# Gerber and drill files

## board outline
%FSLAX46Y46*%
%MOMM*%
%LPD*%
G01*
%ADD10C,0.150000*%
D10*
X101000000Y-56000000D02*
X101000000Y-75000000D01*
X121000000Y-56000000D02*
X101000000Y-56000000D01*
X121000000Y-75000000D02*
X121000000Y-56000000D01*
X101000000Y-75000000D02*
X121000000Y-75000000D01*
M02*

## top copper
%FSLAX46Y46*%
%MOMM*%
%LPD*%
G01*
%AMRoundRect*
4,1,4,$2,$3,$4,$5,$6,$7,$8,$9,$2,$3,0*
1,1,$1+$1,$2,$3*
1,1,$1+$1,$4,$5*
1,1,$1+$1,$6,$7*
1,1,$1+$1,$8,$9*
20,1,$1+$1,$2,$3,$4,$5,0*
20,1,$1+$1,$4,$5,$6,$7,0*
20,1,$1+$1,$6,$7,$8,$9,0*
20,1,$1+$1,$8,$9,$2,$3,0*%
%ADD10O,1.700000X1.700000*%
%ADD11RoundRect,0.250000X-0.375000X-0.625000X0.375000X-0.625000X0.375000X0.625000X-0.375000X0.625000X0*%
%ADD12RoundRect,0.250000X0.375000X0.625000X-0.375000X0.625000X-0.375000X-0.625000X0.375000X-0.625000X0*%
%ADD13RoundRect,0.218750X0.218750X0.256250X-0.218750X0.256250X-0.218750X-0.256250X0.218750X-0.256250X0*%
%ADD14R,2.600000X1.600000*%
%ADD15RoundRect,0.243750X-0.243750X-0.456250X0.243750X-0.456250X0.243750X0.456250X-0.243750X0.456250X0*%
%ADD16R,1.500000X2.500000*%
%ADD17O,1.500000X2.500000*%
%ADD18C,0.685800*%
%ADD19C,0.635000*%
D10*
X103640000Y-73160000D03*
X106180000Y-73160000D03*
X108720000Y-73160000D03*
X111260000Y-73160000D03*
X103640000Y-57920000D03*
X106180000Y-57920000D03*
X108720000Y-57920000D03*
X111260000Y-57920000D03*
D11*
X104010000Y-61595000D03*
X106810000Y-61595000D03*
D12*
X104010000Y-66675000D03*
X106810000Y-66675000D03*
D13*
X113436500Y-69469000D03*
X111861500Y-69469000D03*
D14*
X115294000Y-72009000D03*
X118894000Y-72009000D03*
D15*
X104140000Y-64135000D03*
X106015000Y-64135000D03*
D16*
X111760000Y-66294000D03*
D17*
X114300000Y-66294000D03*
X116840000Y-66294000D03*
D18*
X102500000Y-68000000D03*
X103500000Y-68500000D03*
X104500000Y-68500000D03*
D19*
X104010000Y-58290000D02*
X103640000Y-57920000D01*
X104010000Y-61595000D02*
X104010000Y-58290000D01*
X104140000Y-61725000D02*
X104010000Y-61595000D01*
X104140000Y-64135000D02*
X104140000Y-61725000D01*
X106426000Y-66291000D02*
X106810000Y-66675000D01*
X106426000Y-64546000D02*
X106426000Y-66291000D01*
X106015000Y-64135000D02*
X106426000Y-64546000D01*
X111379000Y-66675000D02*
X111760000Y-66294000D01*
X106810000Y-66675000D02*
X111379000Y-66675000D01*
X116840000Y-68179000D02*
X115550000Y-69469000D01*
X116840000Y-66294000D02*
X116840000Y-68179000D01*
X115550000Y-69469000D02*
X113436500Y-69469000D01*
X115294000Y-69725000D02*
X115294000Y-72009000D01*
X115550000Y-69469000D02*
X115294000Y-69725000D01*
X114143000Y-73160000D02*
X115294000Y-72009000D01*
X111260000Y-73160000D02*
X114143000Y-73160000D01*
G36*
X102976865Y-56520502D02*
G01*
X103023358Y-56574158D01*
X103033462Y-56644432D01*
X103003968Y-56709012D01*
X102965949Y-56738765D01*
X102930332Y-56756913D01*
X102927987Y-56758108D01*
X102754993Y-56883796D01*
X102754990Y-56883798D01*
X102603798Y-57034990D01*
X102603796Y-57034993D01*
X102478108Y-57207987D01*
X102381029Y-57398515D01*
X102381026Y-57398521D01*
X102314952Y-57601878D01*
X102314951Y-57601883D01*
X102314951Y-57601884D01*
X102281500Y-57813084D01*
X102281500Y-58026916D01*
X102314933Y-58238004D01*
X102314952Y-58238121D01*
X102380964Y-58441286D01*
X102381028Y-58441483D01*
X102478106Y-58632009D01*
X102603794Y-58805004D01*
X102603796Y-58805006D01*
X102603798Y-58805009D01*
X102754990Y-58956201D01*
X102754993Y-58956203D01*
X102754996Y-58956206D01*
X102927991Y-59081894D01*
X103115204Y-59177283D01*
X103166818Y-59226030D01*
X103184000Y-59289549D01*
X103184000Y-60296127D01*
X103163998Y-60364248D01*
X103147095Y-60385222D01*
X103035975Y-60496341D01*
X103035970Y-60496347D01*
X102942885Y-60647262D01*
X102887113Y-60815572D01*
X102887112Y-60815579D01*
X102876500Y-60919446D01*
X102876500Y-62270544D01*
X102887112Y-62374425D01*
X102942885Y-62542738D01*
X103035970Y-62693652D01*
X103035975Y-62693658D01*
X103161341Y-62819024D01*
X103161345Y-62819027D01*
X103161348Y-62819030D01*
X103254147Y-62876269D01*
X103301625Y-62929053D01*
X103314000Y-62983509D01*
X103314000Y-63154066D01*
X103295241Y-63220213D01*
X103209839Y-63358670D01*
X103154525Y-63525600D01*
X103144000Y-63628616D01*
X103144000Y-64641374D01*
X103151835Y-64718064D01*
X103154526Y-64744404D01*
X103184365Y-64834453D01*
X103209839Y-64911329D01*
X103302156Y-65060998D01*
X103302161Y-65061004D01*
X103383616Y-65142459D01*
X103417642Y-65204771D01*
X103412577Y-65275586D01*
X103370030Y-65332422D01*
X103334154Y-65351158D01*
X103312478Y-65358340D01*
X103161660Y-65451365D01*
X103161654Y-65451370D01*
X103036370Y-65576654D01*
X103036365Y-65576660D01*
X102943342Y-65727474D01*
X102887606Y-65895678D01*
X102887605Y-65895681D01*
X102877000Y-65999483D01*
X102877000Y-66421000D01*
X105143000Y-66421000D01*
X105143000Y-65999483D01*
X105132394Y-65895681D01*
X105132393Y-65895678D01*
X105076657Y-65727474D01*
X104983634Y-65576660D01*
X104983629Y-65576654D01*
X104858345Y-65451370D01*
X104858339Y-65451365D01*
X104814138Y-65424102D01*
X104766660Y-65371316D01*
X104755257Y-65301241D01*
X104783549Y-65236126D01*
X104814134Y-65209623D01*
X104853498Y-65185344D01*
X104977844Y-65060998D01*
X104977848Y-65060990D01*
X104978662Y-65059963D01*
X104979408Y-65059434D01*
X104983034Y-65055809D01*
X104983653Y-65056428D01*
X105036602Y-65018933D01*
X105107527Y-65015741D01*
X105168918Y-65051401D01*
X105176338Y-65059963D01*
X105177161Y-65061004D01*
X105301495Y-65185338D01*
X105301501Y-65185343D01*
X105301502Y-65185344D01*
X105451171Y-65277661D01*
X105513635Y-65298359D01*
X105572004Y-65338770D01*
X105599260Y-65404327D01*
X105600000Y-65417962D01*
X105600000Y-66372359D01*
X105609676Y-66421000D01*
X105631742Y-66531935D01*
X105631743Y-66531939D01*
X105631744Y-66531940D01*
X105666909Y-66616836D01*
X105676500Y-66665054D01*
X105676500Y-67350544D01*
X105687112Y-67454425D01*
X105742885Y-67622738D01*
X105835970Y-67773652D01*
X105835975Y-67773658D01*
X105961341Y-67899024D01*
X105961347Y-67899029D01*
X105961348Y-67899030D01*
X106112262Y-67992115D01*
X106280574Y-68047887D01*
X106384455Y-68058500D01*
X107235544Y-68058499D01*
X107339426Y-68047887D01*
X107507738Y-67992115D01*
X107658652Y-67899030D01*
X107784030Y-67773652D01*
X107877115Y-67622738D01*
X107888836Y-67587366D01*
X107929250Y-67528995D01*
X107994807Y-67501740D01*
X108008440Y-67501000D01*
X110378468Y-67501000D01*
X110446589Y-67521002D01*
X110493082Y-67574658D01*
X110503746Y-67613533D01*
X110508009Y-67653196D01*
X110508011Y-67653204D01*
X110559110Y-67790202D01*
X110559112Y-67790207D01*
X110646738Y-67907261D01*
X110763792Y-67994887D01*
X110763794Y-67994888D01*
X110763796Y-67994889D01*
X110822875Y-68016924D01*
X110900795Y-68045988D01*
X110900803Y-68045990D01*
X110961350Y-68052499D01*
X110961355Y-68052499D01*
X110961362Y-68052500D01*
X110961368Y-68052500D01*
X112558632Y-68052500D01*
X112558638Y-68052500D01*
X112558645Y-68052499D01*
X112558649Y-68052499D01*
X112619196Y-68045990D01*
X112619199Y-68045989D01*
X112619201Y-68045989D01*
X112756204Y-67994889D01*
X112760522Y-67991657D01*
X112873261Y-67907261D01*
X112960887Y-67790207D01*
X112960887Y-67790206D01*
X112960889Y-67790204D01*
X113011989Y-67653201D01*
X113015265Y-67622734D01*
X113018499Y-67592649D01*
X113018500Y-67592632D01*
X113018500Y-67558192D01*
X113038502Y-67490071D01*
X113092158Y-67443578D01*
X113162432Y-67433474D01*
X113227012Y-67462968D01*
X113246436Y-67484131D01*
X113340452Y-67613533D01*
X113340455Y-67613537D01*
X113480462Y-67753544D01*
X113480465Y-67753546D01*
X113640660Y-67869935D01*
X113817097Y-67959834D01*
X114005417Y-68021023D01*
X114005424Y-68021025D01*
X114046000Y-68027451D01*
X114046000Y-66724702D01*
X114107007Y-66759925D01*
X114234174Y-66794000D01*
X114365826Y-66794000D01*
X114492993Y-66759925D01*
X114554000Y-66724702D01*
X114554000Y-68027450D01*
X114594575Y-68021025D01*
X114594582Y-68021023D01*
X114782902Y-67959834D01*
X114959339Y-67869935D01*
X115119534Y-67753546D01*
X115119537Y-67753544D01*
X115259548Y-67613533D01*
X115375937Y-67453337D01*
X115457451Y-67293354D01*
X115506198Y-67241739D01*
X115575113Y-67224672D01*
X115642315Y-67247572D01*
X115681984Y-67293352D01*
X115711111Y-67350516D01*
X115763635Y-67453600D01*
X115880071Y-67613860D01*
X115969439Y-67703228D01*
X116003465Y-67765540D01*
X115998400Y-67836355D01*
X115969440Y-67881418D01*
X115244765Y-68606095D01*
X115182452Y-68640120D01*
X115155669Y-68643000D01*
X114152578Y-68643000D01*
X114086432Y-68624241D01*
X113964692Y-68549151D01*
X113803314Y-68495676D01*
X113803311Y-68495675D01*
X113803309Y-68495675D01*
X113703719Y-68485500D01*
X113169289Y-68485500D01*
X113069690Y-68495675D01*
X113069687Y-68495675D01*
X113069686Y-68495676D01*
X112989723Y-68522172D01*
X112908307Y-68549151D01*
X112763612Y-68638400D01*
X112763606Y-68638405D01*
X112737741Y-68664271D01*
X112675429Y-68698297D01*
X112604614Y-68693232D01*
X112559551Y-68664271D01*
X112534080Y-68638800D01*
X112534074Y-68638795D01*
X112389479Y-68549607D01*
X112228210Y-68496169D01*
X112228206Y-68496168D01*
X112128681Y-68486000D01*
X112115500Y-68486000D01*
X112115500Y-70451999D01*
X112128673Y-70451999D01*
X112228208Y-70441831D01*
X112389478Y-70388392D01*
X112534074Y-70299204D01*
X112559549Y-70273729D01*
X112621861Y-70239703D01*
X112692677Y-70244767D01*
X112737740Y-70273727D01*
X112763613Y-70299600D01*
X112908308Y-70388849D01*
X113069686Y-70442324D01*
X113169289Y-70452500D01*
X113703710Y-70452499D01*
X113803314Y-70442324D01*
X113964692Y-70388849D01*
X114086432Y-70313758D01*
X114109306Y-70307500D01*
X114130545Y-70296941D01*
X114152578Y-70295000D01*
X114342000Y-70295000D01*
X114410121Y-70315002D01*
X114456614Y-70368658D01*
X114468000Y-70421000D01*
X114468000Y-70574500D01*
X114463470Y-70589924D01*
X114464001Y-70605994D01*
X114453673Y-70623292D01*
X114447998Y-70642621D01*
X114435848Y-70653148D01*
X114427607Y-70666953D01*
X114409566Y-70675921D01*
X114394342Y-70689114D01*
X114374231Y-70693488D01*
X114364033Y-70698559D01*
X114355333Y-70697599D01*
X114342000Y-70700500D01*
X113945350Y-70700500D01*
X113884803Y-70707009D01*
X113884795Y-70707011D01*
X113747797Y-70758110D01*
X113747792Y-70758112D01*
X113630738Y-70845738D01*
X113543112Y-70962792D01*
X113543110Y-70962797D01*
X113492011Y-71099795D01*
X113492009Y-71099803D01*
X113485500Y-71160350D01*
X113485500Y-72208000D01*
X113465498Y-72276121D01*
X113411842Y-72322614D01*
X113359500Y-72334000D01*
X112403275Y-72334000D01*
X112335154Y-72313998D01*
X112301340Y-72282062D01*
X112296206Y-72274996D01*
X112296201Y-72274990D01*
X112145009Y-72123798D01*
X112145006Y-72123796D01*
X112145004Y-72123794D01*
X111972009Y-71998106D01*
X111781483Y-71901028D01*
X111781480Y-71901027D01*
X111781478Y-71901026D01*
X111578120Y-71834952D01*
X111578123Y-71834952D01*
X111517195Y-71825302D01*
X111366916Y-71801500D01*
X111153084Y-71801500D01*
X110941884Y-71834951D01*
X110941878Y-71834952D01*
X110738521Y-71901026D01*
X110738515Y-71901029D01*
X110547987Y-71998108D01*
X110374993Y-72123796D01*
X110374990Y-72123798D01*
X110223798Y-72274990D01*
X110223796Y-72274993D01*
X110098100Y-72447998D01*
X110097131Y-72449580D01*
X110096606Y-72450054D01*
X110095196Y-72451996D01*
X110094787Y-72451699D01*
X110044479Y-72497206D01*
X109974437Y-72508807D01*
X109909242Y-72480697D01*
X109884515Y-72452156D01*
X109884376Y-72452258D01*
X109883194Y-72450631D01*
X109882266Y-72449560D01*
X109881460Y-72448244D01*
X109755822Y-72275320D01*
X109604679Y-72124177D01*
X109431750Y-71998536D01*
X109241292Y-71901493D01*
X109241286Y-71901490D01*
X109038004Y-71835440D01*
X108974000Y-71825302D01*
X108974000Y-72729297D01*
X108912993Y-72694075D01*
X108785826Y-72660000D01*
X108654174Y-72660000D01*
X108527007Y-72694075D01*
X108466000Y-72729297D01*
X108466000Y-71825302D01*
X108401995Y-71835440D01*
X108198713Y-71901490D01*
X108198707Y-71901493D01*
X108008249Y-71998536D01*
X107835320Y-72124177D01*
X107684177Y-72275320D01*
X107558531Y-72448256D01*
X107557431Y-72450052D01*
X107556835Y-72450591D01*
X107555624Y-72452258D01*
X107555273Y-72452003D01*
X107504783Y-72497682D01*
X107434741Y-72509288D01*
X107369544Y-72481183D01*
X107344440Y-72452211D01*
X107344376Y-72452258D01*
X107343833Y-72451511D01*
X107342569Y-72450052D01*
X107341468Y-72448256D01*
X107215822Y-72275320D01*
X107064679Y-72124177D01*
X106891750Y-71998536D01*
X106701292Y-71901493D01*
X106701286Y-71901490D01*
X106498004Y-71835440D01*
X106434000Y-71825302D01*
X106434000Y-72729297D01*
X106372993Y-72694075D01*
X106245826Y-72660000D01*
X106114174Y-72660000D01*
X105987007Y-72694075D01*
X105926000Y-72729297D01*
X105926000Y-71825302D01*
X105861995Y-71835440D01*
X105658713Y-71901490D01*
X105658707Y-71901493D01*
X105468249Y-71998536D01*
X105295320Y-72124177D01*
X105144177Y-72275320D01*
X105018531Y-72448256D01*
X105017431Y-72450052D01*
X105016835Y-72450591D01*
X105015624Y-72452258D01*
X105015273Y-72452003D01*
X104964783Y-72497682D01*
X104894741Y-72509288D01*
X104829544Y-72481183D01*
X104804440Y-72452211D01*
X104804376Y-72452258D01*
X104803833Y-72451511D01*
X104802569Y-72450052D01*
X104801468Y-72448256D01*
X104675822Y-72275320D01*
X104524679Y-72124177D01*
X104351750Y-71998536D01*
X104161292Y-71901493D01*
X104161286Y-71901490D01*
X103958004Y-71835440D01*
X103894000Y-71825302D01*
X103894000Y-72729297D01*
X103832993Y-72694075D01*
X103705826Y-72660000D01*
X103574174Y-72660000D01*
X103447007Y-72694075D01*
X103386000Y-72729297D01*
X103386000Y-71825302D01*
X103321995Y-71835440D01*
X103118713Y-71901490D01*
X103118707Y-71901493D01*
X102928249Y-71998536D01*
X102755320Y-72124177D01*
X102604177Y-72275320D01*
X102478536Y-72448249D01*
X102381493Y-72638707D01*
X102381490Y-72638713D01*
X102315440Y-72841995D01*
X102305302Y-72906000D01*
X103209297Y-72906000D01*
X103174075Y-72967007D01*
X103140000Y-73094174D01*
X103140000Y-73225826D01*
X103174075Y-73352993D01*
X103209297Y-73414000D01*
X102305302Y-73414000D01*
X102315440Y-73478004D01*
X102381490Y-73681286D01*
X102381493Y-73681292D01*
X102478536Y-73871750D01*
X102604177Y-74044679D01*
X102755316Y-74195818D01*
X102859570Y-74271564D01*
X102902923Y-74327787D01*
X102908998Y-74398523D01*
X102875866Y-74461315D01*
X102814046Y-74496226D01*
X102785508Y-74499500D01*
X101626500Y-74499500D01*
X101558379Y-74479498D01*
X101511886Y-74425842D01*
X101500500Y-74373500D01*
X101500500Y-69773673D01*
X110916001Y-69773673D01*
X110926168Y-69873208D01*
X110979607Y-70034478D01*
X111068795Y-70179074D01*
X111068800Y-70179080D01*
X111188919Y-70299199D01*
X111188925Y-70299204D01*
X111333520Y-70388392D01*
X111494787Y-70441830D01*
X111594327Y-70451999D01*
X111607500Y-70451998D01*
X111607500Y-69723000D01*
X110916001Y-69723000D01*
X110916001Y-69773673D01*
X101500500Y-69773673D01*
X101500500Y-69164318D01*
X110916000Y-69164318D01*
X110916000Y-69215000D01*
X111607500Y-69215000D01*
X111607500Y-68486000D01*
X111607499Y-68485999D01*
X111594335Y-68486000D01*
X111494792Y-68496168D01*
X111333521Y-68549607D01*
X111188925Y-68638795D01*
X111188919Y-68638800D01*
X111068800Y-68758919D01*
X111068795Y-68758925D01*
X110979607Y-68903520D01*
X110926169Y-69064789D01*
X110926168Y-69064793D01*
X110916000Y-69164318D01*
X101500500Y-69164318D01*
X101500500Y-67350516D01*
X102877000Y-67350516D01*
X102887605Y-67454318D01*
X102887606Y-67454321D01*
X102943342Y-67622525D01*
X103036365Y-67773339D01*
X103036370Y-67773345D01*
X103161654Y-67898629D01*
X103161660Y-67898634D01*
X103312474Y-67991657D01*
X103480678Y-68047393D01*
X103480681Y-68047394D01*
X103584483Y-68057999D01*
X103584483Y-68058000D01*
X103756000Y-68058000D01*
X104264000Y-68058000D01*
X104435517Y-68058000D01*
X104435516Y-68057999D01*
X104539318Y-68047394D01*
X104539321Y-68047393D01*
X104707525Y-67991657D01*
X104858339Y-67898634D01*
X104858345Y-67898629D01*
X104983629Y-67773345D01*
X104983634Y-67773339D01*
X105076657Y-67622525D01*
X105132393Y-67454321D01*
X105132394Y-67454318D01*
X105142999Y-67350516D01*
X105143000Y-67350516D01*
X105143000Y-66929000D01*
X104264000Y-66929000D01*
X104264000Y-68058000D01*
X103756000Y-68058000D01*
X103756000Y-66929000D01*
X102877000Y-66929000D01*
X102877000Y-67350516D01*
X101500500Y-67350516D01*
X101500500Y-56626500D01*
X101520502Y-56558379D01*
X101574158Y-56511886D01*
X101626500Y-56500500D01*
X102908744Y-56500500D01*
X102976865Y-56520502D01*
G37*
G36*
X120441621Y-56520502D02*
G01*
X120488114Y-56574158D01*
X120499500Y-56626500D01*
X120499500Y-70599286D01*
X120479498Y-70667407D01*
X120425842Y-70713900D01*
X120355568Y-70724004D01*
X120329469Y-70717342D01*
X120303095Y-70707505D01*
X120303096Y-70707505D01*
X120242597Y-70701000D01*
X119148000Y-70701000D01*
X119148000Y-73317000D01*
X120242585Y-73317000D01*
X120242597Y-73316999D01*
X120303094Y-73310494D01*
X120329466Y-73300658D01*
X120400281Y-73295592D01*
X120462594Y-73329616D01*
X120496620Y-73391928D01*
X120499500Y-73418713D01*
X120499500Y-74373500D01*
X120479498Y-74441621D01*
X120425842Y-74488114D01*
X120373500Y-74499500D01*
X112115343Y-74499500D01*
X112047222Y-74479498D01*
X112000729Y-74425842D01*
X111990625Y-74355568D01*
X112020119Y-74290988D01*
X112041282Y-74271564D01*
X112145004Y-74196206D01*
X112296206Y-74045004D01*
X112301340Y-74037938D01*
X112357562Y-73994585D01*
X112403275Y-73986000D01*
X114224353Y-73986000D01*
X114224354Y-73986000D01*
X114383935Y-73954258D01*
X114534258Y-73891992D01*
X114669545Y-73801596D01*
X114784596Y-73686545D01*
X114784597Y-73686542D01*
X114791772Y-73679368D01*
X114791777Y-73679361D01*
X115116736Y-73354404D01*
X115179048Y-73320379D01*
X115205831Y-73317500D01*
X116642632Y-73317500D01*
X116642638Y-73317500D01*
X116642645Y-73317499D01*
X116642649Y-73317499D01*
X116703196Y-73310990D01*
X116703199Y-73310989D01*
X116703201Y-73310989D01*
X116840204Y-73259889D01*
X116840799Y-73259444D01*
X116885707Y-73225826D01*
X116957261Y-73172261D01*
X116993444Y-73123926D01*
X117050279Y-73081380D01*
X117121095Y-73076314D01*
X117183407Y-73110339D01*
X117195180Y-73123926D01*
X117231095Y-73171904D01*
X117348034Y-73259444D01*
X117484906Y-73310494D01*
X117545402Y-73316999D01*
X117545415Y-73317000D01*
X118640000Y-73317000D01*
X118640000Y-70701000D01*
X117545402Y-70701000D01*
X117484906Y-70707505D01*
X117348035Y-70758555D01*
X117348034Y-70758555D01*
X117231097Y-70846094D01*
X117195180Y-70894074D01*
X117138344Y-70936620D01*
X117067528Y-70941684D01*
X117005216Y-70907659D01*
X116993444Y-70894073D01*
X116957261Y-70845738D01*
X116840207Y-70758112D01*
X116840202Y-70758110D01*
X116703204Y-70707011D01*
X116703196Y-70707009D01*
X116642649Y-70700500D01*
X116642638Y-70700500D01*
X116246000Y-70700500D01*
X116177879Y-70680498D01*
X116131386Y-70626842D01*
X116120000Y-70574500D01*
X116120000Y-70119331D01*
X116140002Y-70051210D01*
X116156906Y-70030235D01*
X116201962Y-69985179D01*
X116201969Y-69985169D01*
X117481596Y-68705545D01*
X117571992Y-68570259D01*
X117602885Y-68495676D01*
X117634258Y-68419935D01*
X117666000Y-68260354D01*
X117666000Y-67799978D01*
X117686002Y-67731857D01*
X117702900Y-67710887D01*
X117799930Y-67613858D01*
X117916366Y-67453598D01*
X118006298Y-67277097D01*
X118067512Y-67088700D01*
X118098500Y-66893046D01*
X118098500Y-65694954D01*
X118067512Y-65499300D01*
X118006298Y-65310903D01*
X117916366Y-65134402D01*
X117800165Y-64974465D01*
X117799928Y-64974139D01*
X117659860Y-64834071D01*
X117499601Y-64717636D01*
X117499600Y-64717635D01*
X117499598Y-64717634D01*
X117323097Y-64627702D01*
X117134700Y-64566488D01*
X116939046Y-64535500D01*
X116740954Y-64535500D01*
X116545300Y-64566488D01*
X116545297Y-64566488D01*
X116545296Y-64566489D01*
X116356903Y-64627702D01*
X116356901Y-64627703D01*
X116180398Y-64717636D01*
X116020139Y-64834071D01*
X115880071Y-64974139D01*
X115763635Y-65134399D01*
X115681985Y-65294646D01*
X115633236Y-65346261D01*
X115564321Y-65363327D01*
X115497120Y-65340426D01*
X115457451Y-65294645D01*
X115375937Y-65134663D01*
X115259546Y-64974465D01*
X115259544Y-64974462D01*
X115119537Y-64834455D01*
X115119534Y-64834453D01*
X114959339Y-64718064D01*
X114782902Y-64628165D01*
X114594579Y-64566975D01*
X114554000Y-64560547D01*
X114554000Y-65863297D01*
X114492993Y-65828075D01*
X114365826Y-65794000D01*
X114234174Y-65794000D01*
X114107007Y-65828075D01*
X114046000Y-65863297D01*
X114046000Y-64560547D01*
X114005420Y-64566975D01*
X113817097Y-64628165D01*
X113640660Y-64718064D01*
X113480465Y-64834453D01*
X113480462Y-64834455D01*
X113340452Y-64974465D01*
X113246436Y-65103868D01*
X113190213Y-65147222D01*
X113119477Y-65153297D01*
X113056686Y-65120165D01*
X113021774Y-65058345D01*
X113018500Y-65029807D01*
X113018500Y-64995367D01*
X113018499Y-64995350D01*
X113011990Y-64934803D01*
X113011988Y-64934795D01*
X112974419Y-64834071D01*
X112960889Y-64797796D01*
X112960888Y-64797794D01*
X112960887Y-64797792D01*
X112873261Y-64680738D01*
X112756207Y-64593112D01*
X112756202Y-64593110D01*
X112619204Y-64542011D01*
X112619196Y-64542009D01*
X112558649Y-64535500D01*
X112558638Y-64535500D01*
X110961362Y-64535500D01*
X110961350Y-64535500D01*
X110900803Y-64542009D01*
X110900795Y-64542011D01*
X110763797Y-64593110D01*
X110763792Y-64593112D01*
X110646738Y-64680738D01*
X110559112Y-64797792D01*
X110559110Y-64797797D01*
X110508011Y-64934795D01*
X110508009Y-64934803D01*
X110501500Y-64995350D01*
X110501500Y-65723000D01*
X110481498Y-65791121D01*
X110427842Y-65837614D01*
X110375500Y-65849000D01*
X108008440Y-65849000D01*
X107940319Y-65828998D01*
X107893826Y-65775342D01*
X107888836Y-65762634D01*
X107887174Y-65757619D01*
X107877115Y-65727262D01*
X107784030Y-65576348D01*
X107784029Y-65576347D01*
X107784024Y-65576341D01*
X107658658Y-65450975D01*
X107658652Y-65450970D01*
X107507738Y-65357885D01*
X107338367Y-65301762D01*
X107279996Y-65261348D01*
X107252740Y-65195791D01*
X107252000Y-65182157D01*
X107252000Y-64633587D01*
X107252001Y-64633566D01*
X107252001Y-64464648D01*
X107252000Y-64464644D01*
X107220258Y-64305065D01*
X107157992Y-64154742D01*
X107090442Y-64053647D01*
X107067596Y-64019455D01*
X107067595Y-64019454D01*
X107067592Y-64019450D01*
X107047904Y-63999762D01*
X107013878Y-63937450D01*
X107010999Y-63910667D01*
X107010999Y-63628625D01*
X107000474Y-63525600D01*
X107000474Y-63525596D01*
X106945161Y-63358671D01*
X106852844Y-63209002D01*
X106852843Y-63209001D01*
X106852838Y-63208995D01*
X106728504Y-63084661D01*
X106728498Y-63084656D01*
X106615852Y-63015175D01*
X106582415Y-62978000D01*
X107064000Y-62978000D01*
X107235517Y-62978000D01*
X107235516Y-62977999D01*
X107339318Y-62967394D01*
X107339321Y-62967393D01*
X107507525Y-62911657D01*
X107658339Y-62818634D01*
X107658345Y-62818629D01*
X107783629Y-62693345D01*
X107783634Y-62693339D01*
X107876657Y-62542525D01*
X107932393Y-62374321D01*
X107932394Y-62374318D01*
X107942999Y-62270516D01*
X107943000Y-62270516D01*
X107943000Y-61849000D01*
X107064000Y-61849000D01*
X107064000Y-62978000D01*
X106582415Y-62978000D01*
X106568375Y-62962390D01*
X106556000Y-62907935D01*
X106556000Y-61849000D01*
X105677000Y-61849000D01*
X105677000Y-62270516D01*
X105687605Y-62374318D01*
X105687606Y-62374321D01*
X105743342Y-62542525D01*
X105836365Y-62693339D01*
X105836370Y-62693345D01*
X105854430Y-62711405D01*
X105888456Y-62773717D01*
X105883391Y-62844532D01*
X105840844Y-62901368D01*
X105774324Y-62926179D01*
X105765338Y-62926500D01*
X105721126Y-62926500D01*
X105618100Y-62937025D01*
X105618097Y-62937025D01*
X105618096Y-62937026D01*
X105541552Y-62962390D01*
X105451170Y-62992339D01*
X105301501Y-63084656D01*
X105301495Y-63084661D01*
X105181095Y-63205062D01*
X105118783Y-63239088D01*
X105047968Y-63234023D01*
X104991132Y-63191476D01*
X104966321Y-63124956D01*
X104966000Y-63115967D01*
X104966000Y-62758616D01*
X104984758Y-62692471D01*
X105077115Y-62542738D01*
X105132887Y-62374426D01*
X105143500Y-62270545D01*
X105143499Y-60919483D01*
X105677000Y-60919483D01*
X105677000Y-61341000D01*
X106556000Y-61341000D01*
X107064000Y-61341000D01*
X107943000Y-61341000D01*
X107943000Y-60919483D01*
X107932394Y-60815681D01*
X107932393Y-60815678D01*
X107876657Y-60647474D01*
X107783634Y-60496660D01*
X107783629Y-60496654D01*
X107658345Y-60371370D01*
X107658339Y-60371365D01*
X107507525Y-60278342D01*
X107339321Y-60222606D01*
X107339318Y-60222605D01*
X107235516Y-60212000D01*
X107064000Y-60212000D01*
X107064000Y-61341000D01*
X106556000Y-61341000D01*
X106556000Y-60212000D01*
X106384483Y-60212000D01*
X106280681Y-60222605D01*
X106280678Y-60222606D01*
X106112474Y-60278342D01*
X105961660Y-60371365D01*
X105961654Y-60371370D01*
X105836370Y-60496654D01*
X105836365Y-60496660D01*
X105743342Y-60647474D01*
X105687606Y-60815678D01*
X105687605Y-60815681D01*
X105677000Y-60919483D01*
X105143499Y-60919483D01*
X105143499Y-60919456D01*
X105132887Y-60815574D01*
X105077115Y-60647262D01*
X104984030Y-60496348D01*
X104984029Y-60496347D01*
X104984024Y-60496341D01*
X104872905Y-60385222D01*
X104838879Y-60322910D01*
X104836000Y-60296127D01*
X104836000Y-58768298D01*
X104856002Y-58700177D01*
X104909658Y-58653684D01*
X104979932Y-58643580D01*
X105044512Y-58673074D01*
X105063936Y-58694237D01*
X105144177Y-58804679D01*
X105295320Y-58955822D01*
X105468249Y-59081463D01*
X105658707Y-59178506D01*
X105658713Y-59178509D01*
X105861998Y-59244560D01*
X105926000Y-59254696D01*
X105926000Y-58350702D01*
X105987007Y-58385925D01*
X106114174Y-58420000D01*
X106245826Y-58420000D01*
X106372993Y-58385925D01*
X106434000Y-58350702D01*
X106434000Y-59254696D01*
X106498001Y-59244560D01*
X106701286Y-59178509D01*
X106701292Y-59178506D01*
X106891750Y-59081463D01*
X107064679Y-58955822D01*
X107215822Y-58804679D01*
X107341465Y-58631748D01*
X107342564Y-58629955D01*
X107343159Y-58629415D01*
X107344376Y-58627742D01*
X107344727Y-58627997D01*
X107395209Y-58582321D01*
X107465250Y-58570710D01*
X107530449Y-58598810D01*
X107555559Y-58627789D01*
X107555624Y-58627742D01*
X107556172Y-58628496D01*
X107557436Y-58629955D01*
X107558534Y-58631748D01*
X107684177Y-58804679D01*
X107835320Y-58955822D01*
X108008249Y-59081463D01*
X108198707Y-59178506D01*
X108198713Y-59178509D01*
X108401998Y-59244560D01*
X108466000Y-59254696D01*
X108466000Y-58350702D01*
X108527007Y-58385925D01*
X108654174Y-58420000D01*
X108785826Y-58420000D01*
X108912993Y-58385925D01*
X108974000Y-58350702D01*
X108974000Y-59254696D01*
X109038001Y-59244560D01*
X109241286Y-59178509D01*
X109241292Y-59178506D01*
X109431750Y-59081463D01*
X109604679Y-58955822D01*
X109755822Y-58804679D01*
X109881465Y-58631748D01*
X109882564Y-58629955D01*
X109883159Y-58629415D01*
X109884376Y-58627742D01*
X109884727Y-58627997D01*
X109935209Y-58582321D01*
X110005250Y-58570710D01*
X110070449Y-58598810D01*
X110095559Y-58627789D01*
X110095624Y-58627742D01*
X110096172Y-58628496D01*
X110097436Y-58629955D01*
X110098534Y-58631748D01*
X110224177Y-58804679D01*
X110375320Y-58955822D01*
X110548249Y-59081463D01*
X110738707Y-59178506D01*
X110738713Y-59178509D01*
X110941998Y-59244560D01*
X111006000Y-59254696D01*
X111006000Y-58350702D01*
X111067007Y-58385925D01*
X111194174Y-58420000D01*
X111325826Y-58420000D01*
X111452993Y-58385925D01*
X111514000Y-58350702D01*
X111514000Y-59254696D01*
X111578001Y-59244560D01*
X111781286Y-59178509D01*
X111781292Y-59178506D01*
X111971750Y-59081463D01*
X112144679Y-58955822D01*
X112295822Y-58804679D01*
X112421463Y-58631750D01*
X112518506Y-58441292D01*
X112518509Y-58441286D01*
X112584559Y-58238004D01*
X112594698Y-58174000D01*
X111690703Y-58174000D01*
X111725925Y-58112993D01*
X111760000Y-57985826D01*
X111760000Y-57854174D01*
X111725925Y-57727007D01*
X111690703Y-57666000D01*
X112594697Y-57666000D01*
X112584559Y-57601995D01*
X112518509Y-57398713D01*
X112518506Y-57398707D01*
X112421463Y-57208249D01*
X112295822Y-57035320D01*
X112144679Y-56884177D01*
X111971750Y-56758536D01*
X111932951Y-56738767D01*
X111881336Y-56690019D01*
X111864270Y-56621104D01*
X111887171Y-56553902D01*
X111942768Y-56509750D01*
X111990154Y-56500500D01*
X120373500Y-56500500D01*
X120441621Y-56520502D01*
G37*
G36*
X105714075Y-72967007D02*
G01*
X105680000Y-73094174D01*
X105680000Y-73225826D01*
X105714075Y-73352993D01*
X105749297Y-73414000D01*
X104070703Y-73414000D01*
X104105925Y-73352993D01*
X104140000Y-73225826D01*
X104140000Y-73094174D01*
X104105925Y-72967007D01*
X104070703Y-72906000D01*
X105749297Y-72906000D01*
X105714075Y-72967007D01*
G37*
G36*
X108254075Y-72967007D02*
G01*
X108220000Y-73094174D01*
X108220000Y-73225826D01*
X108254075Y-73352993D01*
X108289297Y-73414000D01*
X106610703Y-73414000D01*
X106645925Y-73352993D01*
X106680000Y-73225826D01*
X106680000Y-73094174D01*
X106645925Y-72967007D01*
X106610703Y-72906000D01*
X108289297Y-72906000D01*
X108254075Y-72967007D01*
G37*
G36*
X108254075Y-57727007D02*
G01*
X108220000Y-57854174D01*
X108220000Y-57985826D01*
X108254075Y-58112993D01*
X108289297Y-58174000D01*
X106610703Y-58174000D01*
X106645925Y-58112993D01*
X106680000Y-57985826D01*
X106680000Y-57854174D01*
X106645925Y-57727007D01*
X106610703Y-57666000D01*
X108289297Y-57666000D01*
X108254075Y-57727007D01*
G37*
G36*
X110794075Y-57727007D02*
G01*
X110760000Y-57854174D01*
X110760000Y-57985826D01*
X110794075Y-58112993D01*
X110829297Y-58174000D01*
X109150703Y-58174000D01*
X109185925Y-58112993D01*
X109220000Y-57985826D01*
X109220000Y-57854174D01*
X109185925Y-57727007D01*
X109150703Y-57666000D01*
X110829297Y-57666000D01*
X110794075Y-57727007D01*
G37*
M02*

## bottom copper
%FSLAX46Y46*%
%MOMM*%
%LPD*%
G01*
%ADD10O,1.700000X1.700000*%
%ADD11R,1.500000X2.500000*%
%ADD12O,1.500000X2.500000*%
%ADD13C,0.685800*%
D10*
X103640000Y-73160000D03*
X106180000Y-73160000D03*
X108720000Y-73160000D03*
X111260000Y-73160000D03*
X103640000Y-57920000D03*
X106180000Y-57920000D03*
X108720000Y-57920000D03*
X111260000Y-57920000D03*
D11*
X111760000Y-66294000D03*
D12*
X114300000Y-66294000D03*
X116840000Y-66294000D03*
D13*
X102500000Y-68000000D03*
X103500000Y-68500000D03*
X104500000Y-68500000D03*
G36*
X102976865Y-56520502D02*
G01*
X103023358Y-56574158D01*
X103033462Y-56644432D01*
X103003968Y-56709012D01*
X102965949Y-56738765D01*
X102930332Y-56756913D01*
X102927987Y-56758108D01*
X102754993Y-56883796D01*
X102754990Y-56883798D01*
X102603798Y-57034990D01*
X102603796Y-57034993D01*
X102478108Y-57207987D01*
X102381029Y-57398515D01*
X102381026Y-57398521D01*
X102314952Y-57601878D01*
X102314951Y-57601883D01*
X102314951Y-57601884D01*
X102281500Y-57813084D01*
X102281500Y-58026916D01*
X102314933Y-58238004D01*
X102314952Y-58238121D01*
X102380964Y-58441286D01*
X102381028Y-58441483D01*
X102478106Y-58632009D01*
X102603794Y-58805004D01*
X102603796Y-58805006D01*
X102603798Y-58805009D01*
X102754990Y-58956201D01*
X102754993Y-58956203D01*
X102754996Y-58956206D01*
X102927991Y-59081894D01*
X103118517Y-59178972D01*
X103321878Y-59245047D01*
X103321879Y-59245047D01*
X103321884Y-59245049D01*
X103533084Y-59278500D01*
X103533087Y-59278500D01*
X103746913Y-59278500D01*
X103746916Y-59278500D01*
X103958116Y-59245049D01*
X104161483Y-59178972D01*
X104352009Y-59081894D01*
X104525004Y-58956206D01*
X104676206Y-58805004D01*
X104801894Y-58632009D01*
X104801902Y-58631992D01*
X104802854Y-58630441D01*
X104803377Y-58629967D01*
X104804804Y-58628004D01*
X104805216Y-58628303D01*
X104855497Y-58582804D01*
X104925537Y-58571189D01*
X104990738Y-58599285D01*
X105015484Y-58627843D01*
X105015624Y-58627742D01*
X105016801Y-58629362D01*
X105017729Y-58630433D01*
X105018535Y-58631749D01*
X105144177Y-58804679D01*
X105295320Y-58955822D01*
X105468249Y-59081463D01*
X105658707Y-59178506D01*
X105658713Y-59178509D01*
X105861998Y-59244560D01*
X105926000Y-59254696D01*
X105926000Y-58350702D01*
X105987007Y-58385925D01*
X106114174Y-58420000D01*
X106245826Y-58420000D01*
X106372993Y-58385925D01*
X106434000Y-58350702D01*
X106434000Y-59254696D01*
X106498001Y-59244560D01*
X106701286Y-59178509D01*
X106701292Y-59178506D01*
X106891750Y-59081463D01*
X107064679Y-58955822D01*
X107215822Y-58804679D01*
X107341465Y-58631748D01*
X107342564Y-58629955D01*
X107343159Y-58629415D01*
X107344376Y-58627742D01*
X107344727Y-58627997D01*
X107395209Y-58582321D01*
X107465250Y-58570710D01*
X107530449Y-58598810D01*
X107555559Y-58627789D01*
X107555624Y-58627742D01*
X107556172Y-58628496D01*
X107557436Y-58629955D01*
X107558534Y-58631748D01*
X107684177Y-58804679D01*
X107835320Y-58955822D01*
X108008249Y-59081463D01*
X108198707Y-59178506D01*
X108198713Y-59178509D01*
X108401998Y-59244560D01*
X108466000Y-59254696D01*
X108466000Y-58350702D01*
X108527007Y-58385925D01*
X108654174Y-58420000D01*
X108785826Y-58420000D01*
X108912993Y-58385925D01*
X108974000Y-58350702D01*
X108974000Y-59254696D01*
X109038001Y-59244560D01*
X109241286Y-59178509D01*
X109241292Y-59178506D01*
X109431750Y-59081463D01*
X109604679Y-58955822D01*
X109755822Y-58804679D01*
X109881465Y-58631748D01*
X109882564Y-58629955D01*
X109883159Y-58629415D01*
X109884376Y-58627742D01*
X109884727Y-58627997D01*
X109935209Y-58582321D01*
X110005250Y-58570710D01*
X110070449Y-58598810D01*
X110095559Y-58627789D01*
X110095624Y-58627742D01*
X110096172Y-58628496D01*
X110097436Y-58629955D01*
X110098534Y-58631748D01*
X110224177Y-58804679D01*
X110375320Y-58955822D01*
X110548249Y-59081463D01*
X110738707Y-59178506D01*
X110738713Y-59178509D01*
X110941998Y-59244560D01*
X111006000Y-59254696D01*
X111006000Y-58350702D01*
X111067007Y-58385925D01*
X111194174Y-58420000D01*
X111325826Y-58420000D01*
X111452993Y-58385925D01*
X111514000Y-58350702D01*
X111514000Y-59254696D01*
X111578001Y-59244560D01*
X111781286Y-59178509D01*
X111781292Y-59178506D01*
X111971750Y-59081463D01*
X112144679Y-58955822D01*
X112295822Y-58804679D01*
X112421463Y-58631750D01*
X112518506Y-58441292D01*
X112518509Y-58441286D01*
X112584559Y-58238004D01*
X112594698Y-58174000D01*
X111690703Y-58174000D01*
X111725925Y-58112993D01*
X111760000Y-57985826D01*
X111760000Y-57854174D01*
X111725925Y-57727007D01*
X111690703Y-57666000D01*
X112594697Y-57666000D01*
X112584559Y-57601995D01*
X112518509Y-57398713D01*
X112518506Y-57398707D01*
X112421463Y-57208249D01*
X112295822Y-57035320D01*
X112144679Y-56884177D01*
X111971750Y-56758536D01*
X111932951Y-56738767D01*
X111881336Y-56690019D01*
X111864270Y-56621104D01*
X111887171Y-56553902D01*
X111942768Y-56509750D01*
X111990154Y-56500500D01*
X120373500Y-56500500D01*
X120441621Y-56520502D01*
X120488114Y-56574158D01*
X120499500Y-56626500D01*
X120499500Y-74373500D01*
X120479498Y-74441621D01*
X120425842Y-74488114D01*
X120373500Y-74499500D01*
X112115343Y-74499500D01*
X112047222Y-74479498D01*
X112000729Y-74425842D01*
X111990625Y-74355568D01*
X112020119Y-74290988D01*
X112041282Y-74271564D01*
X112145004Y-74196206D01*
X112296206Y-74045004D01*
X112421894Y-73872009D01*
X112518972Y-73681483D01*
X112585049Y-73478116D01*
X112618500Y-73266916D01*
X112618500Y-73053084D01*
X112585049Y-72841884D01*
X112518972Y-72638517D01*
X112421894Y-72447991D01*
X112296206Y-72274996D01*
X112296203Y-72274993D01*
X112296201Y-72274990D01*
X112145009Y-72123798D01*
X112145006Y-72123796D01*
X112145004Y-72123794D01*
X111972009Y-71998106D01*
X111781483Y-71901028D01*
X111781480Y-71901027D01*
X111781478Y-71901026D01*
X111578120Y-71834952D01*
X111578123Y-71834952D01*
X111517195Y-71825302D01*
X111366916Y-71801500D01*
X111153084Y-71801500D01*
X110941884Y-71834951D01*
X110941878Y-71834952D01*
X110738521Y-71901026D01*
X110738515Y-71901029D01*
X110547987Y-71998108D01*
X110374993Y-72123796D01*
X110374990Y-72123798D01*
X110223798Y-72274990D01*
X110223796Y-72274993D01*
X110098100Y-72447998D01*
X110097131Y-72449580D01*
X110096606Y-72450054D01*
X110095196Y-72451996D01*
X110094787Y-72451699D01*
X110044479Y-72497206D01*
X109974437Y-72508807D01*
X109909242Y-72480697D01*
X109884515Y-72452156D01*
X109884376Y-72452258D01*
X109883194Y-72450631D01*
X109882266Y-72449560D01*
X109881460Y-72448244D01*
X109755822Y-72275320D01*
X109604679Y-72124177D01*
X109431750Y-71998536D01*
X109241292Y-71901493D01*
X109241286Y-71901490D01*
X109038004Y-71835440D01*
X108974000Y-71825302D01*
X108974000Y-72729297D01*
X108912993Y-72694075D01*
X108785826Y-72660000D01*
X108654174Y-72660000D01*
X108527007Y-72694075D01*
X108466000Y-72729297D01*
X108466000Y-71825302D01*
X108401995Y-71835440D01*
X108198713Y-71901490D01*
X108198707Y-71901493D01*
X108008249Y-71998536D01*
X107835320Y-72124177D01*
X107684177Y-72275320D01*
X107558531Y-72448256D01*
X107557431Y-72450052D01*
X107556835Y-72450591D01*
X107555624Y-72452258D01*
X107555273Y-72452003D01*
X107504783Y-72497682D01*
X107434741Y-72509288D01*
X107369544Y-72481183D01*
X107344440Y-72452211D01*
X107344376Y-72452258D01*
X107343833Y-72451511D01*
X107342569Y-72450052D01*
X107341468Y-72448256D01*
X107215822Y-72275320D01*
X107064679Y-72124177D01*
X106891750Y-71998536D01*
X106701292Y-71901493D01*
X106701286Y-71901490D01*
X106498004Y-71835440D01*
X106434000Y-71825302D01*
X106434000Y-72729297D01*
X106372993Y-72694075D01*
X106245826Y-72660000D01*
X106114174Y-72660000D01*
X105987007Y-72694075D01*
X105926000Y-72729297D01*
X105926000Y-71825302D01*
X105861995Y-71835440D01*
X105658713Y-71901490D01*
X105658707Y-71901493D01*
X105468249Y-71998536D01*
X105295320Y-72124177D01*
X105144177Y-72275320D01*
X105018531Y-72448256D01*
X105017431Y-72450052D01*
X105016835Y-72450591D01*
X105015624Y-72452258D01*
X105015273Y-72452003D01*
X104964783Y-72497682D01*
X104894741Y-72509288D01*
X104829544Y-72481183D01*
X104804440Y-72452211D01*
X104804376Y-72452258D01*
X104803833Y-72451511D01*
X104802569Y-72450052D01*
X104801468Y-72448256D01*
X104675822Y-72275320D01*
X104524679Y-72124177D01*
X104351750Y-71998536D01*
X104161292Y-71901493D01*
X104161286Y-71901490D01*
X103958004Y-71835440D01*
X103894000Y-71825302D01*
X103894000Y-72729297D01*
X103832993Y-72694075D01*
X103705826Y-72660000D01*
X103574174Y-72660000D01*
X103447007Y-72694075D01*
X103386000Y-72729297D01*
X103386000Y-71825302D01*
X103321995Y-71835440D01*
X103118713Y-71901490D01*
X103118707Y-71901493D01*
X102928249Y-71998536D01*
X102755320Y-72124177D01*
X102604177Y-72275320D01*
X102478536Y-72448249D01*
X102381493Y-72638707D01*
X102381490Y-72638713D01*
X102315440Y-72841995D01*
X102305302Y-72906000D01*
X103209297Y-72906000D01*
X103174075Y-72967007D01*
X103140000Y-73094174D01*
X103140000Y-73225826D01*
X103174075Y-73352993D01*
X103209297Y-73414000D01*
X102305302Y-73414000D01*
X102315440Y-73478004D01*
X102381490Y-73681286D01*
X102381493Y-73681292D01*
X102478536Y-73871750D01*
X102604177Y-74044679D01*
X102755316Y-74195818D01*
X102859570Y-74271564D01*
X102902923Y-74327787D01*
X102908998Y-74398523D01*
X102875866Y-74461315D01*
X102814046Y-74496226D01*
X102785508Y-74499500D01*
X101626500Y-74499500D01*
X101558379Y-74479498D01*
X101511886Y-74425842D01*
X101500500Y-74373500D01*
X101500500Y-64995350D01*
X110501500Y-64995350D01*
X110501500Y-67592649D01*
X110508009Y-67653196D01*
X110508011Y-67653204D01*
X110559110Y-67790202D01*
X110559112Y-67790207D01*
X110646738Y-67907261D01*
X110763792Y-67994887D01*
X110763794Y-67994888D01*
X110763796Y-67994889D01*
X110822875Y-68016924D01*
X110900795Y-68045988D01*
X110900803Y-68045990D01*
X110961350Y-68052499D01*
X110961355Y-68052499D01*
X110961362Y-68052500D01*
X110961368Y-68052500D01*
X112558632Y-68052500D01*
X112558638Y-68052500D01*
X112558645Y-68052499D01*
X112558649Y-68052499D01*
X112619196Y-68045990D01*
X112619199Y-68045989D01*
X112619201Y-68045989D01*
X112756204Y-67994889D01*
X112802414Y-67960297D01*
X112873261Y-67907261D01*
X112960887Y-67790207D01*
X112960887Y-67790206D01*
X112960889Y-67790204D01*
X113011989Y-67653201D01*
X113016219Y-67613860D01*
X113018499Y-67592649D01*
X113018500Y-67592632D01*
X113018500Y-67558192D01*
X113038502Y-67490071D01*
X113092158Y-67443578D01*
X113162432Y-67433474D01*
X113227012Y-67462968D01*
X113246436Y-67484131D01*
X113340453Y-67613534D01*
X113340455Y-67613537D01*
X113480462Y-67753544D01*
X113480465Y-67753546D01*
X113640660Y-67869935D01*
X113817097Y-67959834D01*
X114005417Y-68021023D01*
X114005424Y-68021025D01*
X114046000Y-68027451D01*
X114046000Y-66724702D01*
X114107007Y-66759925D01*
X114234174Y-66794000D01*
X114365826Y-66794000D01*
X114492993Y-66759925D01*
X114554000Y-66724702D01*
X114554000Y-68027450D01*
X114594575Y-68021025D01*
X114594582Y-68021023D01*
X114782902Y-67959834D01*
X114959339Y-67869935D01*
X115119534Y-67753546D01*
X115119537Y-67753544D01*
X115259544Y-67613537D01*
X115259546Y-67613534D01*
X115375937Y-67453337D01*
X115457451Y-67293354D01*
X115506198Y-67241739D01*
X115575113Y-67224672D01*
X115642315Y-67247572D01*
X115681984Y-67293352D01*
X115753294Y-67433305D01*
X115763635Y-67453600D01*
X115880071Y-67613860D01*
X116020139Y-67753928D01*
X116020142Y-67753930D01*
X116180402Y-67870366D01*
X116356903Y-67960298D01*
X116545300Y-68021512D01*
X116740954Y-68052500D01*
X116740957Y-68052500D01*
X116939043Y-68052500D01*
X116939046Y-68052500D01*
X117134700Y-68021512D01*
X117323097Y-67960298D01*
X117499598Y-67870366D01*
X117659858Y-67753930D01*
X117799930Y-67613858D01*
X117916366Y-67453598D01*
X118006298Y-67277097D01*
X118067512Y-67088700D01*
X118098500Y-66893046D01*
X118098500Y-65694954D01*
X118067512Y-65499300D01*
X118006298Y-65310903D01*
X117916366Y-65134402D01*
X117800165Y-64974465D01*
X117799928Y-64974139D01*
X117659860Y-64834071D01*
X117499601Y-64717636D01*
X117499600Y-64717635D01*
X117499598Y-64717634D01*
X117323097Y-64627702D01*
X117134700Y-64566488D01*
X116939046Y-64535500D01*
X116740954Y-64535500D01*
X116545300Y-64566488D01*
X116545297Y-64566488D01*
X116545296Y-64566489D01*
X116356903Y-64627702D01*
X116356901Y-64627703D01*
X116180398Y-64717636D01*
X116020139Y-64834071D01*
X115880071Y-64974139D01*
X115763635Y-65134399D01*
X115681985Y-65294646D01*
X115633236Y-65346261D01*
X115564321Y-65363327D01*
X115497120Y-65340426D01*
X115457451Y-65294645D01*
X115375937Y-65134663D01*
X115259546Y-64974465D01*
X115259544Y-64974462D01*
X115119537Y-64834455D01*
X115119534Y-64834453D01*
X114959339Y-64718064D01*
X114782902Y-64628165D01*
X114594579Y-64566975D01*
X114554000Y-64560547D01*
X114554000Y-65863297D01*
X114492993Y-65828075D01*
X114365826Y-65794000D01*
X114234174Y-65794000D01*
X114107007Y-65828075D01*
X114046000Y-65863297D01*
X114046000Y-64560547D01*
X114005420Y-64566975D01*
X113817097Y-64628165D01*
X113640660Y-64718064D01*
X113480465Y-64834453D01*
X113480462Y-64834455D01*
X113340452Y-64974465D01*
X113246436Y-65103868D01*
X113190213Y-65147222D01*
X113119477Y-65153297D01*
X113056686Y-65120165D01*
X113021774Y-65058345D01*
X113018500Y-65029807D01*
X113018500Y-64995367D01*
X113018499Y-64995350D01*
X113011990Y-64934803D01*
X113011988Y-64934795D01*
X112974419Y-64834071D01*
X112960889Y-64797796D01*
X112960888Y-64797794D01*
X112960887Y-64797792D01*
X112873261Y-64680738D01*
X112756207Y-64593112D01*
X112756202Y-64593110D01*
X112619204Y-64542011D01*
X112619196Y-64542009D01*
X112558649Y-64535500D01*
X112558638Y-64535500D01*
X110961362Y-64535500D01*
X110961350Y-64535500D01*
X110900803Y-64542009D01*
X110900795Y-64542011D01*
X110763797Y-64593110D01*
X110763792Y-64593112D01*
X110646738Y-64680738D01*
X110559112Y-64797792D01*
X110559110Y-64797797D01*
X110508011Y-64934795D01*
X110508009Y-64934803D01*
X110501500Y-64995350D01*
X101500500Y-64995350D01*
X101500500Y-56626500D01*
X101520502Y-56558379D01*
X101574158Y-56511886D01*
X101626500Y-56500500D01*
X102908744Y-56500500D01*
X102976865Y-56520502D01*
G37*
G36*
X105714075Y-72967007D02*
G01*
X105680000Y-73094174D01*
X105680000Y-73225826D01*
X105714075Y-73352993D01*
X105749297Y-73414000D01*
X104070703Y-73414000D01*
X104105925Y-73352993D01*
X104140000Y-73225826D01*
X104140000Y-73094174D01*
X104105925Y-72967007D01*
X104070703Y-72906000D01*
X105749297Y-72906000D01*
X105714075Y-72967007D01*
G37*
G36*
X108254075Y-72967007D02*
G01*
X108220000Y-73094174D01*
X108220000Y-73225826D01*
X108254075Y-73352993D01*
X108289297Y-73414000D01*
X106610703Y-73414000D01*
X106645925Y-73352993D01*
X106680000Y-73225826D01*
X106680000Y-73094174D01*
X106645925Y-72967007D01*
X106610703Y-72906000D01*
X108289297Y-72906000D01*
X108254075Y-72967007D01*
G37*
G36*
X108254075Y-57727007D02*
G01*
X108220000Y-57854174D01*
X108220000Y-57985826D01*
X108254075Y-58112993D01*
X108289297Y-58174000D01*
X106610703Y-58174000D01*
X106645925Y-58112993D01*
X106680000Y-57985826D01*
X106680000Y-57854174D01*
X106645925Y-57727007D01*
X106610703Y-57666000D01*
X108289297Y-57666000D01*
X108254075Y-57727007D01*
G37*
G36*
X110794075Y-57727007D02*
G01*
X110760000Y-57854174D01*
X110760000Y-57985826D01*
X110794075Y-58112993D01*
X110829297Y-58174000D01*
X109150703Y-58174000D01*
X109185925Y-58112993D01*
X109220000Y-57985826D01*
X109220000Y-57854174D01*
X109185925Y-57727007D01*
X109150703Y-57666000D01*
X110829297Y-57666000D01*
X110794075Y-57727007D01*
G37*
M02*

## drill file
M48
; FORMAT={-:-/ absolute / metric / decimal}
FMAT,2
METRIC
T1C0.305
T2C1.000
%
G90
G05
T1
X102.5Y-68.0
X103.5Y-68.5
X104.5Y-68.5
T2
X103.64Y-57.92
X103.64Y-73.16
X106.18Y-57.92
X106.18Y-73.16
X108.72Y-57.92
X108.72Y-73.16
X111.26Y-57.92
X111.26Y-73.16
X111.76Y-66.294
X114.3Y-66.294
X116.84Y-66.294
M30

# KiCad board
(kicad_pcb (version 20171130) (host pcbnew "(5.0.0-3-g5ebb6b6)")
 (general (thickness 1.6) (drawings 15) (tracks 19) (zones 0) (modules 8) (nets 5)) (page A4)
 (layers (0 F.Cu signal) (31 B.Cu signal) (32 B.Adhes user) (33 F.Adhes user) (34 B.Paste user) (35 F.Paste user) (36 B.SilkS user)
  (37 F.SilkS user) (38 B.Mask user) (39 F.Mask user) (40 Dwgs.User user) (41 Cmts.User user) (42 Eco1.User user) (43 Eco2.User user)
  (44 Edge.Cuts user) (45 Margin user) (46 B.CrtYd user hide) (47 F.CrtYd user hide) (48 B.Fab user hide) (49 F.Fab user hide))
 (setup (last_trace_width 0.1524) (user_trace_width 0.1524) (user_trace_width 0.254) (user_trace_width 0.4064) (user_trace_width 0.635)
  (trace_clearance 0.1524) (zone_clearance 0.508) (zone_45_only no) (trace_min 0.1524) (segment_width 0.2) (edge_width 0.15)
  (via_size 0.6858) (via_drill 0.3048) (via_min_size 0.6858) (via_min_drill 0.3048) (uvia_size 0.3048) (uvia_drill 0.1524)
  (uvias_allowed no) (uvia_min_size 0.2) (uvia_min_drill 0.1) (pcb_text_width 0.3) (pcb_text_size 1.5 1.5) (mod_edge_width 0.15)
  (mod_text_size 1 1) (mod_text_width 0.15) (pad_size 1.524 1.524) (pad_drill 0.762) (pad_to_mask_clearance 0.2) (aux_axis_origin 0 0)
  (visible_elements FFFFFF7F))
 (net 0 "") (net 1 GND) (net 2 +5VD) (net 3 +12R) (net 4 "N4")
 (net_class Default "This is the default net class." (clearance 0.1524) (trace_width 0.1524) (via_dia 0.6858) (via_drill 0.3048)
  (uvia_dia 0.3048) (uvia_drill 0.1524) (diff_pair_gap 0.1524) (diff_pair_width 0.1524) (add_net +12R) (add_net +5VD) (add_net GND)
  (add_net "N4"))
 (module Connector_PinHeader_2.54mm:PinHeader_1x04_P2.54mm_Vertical (layer B.Cu) (at 111.26 73.16 90)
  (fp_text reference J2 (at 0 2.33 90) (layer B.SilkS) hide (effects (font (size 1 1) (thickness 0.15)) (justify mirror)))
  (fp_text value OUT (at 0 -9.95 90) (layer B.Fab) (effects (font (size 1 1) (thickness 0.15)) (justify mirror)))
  (pad 4 thru_hole oval (at 0 -7.62 90) (size 1.7 1.7) (drill 1) (layers *.Cu *.Mask) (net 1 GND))
  (pad 3 thru_hole oval (at 0 -5.08 90) (size 1.7 1.7) (drill 1) (layers *.Cu *.Mask) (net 1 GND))
  (pad 2 thru_hole oval (at 0 -2.54 90) (size 1.7 1.7) (drill 1) (layers *.Cu *.Mask) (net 1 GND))
  (pad 1 thru_hole oval (at 0 0 90) (size 1.7 1.7) (drill 1) (layers *.Cu *.Mask) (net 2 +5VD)))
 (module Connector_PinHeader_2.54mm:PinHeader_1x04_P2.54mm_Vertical (layer B.Cu) (at 103.64 57.92 270)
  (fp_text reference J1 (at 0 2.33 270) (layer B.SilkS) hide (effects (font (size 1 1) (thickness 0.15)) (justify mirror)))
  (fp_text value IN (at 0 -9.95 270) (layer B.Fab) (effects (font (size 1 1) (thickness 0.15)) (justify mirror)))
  (pad 1 thru_hole oval (at 0 0 270) (size 1.7 1.7) (drill 1) (layers *.Cu *.Mask) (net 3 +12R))
  (pad 2 thru_hole oval (at 0 -2.54 270) (size 1.7 1.7) (drill 1) (layers *.Cu *.Mask) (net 1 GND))
  (pad 3 thru_hole oval (at 0 -5.08 270) (size 1.7 1.7) (drill 1) (layers *.Cu *.Mask) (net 1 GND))
  (pad 4 thru_hole oval (at 0 -7.62 270) (size 1.7 1.7) (drill 1) (layers *.Cu *.Mask) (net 1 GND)))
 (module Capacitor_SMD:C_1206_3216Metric (layer F.Cu) (at 105.41 61.595)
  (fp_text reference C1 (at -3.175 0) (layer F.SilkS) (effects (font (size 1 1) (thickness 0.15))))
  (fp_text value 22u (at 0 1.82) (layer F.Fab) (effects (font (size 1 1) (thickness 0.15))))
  (pad 1 smd roundrect (at -1.4 0) (size 1.25 1.75) (layers F.Cu F.Paste F.Mask) (roundrect_rratio 0.2) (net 3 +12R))
  (pad 2 smd roundrect (at 1.4 0) (size 1.25 1.75) (layers F.Cu F.Paste F.Mask) (roundrect_rratio 0.2) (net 1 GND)))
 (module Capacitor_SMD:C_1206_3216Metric (layer F.Cu) (at 105.41 66.675 180)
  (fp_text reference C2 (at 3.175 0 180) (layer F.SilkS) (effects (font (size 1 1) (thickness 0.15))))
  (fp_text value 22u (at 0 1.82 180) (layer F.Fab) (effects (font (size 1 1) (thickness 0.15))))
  (pad 2 smd roundrect (at 1.4 0 180) (size 1.25 1.75) (layers F.Cu F.Paste F.Mask) (roundrect_rratio 0.2) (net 1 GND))
  (pad 1 smd roundrect (at -1.4 0 180) (size 1.25 1.75) (layers F.Cu F.Paste F.Mask) (roundrect_rratio 0.2) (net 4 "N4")))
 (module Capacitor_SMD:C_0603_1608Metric (layer F.Cu) (at 112.649 69.469 180)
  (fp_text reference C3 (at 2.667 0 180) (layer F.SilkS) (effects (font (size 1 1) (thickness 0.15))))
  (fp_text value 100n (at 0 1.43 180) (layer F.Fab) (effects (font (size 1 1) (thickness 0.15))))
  (pad 1 smd roundrect (at -0.7875 0 180) (size 0.875 0.95) (layers F.Cu F.Paste F.Mask) (roundrect_rratio 0.25) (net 2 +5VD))
  (pad 2 smd roundrect (at 0.7875 0 180) (size 0.875 0.95) (layers F.Cu F.Paste F.Mask) (roundrect_rratio 0.25) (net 1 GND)))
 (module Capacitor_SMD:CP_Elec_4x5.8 (layer F.Cu) (at 117.094 72.009)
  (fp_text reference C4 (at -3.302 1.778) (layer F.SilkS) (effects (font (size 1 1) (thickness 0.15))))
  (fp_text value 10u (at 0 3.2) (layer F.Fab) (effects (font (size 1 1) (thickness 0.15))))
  (pad 1 smd rect (at -1.8 0) (size 2.6 1.6) (layers F.Cu F.Paste F.Mask) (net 2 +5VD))
  (pad 2 smd rect (at 1.8 0) (size 2.6 1.6) (layers F.Cu F.Paste F.Mask) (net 1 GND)))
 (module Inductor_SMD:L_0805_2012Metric (layer F.Cu) (at 105.0775 64.135)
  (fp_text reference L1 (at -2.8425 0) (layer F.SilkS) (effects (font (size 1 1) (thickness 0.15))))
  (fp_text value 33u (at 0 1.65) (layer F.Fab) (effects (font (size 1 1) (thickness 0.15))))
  (pad 1 smd roundrect (at -0.9375 0) (size 0.975 1.4) (layers F.Cu F.Paste F.Mask) (roundrect_rratio 0.25) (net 3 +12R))
  (pad 2 smd roundrect (at 0.9375 0) (size 0.975 1.4) (layers F.Cu F.Paste F.Mask) (roundrect_rratio 0.25) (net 4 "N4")))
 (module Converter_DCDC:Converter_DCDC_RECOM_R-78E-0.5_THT (layer F.Cu) (at 111.76 66.294)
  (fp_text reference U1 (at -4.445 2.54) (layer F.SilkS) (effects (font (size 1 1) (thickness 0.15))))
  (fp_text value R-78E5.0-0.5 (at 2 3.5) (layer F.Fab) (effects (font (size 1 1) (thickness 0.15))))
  (pad 1 thru_hole rect (at 0 0) (size 1.5 2.5) (drill 1) (layers *.Cu *.Mask) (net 4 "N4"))
  (pad 2 thru_hole oval (at 2.54 0) (size 1.5 2.5) (drill 1) (layers *.Cu *.Mask) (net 1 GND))
  (pad 3 thru_hole oval (at 5.08 0) (size 1.5 2.5) (drill 1) (layers *.Cu *.Mask) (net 2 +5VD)))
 (gr_line (start 101 56) (end 101 75) (layer Edge.Cuts) (width 0.15))
 (gr_line (start 121 56) (end 101 56) (layer Edge.Cuts) (width 0.15))
 (gr_line (start 121 75) (end 121 56) (layer Edge.Cuts) (width 0.15))
 (gr_line (start 101 75) (end 121 75) (layer Edge.Cuts) (width 0.15))
 (via (at 102.5 68) (size 0.6858) (drill 0.3048) (layers F.Cu B.Cu) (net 1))
 (via (at 103.5 68.5) (size 0.6858) (drill 0.3048) (layers F.Cu B.Cu) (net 1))
 (via (at 104.5 68.5) (size 0.6858) (drill 0.3048) (layers F.Cu B.Cu) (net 1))
 (segment (start 104.01 58.29) (end 103.64 57.92) (width 0.635) (layer F.Cu) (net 3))
 (segment (start 104.01 61.595) (end 104.01 58.29) (width 0.635) (layer F.Cu) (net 3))
 (segment (start 104.14 61.725) (end 104.01 61.595) (width 0.635) (layer F.Cu) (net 3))
 (segment (start 104.14 64.135) (end 104.14 61.725) (width 0.635) (layer F.Cu) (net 3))
 (segment (start 106.426 66.291) (end 106.81 66.675) (width 0.635) (layer F.Cu) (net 4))
 (segment (start 106.426 64.546) (end 106.426 66.291) (width 0.635) (layer F.Cu) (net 4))
 (segment (start 106.015 64.135) (end 106.426 64.546) (width 0.635) (layer F.Cu) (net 4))
 (segment (start 111.379 66.675) (end 111.76 66.294) (width 0.635) (layer F.Cu) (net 4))
 (segment (start 106.81 66.675) (end 111.379 66.675) (width 0.635) (layer F.Cu) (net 4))
 (segment (start 116.84 68.179) (end 115.55 69.469) (width 0.635) (layer F.Cu) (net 2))
 (segment (start 116.84 66.294) (end 116.84 68.179) (width 0.635) (layer F.Cu) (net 2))
 (segment (start 115.55 69.469) (end 113.4365 69.469) (width 0.635) (layer F.Cu) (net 2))
 (segment (start 115.294 69.725) (end 115.294 72.009) (width 0.635) (layer F.Cu) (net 2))
 (segment (start 115.55 69.469) (end 115.294 69.725) (width 0.635) (layer F.Cu) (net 2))
 (segment (start 114.143 73.16) (end 115.294 72.009) (width 0.635) (layer F.Cu) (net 2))
 (segment (start 111.26 73.16) (end 114.143 73.16) (width 0.635) (layer F.Cu) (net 2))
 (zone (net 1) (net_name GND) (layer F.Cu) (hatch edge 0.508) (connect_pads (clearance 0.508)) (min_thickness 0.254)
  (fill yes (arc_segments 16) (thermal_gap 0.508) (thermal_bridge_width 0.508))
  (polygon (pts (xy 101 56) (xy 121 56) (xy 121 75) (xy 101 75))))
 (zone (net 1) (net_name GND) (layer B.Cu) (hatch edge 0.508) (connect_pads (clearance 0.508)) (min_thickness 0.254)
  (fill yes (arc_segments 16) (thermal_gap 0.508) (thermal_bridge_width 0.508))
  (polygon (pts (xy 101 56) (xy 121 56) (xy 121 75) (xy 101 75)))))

